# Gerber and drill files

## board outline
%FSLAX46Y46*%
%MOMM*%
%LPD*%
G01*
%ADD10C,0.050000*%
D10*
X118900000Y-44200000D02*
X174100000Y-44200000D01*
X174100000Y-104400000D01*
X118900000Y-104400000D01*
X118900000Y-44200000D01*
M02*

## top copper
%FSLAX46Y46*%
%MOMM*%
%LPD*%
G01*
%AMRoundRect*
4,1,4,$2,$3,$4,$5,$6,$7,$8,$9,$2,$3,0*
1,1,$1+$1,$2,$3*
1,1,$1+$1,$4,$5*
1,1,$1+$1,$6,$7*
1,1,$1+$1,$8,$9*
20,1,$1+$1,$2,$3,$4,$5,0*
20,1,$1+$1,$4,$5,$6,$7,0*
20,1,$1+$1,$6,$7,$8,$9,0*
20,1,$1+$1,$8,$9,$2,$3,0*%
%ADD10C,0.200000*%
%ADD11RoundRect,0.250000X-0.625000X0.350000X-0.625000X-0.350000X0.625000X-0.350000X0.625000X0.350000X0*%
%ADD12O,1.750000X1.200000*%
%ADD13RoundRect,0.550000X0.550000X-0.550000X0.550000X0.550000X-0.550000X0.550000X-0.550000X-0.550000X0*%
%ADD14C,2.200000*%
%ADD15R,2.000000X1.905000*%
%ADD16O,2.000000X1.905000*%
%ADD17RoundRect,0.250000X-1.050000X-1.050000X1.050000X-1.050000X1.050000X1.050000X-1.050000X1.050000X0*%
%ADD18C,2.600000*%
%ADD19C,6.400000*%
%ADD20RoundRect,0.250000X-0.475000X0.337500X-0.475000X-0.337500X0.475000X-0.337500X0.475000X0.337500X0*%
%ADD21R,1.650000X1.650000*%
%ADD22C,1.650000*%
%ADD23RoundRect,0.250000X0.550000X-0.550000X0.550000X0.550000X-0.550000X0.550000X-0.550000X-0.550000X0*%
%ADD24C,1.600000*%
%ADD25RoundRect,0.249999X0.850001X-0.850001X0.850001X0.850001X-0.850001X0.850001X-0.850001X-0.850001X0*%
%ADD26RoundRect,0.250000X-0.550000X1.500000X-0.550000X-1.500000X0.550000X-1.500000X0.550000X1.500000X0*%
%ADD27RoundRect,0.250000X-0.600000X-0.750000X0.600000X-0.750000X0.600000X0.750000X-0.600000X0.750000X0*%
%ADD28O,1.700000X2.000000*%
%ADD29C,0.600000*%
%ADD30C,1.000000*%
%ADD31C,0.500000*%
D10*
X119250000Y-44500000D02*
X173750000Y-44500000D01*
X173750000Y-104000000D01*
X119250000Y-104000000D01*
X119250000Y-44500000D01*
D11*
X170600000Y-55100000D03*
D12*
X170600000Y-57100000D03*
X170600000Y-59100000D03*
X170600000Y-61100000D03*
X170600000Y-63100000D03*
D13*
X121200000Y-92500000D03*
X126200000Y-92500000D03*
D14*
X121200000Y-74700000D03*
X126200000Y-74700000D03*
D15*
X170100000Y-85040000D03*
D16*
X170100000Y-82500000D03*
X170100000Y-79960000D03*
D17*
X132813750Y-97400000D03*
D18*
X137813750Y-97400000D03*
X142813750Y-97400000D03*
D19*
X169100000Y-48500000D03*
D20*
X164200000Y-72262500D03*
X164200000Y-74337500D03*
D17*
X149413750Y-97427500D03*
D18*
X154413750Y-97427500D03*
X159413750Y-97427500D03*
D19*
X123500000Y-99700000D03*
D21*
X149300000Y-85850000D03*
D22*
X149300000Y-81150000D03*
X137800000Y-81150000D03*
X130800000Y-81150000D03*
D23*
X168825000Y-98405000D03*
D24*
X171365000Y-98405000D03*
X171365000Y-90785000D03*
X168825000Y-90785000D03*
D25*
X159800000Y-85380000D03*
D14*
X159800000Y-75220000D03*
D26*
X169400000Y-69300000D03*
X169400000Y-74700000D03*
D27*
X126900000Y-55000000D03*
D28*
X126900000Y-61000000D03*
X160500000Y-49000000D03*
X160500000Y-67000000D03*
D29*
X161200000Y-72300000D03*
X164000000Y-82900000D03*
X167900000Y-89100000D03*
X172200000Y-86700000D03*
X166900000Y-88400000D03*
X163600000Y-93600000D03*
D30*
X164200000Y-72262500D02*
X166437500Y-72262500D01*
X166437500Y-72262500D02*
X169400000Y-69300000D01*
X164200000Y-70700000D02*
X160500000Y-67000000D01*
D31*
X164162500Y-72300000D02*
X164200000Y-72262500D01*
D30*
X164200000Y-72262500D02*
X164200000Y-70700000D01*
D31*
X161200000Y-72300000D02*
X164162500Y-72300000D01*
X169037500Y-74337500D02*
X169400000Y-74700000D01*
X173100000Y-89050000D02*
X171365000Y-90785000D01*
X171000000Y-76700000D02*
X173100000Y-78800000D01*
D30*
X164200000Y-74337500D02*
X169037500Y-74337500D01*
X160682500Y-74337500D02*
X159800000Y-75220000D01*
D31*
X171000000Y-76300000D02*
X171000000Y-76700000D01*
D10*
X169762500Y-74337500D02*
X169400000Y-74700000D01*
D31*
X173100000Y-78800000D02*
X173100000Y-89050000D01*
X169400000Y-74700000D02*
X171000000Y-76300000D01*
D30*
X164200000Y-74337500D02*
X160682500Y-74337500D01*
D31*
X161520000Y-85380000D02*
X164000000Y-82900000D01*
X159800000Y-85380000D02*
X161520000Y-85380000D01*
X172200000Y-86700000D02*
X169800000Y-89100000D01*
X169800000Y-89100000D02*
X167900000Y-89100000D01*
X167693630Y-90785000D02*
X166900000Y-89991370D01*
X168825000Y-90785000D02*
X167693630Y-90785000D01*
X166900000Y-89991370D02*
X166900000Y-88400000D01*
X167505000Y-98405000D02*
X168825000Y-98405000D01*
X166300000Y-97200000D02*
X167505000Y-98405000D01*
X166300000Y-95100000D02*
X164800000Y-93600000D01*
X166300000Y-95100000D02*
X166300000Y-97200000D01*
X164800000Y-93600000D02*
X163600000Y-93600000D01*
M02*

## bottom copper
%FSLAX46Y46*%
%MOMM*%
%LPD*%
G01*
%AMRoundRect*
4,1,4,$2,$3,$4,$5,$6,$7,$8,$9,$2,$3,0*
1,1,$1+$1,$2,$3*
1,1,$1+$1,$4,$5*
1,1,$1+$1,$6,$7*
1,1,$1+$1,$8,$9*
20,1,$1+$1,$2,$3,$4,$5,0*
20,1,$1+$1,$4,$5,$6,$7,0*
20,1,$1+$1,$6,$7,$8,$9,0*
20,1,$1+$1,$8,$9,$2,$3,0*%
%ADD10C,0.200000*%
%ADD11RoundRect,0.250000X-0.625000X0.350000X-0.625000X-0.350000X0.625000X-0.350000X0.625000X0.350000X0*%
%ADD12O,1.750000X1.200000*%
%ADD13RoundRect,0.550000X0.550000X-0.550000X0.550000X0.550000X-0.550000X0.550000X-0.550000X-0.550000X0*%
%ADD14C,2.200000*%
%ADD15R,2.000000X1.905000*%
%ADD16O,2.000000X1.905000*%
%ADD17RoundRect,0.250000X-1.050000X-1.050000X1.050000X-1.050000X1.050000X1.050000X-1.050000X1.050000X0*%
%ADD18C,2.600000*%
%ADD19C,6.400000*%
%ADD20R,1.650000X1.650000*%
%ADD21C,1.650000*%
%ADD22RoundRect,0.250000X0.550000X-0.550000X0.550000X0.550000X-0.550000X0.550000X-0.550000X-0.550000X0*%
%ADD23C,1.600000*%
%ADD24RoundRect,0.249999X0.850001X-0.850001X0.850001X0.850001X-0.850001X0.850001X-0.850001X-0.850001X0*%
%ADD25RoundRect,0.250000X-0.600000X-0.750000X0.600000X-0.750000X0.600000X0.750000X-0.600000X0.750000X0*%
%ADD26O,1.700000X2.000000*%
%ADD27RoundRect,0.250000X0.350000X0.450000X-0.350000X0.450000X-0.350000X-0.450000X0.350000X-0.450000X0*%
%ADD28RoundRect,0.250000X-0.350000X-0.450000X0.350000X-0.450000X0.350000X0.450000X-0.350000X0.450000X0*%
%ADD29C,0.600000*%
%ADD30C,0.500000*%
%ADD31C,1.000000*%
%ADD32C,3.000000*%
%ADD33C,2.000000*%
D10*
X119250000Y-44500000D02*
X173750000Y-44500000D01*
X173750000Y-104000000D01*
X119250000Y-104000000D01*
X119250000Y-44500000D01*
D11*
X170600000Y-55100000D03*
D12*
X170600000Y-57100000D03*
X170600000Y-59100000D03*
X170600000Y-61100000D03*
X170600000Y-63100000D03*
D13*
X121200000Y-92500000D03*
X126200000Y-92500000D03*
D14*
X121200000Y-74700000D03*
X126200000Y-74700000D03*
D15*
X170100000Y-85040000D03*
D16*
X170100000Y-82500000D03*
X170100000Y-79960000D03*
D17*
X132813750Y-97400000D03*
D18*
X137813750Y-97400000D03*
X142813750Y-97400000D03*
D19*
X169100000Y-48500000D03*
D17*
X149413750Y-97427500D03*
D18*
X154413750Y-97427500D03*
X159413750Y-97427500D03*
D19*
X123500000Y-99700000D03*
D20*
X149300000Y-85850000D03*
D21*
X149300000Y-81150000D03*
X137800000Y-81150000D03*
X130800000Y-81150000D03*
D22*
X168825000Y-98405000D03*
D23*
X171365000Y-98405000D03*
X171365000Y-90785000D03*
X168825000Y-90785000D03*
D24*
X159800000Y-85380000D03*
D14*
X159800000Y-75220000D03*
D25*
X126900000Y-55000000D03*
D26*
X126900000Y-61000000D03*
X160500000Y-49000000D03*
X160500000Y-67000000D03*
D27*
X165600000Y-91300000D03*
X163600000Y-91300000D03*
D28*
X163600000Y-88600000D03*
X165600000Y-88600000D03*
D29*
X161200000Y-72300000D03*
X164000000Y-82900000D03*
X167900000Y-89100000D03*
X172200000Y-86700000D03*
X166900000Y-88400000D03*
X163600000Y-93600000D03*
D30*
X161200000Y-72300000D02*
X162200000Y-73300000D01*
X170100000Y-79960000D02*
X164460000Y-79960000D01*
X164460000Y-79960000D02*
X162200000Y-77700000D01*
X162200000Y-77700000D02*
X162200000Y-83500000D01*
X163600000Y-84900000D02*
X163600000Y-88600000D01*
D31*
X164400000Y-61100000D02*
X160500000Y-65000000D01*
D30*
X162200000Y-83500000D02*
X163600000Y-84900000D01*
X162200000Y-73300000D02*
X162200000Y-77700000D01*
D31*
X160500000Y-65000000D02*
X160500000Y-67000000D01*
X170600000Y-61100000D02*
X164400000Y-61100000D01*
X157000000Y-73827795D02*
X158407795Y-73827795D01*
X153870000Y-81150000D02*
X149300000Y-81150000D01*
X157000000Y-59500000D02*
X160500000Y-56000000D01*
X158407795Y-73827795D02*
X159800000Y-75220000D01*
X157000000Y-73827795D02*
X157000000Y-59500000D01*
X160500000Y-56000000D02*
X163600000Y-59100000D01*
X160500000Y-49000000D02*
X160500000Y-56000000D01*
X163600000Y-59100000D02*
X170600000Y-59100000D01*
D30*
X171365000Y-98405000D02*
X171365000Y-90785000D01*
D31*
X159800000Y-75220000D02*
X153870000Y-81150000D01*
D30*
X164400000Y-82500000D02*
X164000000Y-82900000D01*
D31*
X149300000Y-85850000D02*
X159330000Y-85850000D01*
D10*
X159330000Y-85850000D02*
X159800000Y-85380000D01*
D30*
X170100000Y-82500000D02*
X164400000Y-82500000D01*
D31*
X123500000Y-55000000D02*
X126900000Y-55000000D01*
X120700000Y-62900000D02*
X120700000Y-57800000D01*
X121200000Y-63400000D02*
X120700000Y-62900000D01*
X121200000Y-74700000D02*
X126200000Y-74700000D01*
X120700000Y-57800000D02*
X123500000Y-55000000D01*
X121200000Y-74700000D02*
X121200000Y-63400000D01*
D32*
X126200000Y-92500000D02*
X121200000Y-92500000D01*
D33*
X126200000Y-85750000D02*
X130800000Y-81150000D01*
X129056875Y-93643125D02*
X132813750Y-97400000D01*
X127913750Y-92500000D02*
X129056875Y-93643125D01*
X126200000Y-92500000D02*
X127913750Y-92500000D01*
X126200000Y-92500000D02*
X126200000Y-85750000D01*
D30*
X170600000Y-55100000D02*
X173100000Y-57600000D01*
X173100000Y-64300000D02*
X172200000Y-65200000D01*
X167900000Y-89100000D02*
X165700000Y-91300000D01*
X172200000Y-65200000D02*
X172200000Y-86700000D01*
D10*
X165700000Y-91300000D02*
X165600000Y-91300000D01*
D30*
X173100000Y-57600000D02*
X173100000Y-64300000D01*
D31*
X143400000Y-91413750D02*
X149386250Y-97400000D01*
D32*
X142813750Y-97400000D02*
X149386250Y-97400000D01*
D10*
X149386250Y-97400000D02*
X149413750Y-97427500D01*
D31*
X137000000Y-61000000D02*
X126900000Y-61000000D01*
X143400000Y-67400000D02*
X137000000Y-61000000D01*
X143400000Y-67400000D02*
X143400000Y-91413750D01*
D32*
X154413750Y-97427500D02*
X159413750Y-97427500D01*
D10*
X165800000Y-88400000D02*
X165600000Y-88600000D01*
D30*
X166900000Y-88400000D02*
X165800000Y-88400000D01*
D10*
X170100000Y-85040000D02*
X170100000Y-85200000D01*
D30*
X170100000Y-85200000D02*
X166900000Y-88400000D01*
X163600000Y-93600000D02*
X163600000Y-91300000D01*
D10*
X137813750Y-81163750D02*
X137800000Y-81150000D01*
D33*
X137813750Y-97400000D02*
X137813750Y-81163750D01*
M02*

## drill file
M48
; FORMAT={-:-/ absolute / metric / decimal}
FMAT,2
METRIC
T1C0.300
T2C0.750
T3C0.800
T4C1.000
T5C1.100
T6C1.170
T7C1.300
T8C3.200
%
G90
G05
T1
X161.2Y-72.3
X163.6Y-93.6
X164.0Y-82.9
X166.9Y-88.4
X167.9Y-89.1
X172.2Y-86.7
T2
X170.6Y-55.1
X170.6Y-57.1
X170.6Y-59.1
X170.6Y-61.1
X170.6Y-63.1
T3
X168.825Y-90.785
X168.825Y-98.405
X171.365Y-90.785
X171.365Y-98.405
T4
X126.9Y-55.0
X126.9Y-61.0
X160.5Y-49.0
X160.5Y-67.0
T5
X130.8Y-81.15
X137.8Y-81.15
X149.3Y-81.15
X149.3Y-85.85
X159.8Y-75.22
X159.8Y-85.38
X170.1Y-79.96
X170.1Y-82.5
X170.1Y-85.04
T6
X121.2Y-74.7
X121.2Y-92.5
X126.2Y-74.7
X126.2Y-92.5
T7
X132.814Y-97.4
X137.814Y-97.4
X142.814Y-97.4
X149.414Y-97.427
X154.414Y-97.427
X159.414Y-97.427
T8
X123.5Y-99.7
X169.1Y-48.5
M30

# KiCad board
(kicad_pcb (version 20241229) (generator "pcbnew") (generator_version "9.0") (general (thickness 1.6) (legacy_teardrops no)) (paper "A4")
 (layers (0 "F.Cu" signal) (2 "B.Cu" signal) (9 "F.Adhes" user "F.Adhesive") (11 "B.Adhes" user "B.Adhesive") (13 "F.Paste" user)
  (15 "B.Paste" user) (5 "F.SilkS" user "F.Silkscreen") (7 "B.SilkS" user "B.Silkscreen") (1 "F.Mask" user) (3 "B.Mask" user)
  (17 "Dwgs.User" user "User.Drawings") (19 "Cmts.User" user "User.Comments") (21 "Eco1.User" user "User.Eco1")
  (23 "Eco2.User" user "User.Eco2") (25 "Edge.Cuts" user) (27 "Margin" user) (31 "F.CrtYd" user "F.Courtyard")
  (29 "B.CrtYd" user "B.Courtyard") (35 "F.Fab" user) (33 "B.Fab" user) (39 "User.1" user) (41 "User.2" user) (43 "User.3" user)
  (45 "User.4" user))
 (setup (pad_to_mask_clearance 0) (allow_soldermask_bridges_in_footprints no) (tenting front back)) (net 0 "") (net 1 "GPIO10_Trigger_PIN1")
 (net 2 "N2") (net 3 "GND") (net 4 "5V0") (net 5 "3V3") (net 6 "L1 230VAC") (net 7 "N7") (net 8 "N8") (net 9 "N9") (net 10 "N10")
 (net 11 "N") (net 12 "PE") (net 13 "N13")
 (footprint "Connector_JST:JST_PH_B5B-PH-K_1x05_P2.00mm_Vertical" (layer "F.Cu") (at 170.6 55.1 -90)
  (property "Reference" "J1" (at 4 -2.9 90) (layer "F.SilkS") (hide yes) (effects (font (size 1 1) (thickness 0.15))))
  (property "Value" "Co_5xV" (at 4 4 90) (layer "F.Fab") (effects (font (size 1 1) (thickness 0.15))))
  (pad "1" thru_hole roundrect (at 0 0 270) (size 1.2 1.75) (drill 0.75) (layers "*.Cu" "*.Mask") (remove_unused_layers no)
   (roundrect_rratio 0.208333) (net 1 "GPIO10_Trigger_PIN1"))
  (pad "2" thru_hole oval (at 2 0 270) (size 1.2 1.75) (drill 0.75) (layers "*.Cu" "*.Mask") (remove_unused_layers no) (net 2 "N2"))
  (pad "3" thru_hole oval (at 4 0 270) (size 1.2 1.75) (drill 0.75) (layers "*.Cu" "*.Mask") (remove_unused_layers no) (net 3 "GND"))
  (pad "4" thru_hole oval (at 6 0 270) (size 1.2 1.75) (drill 0.75) (layers "*.Cu" "*.Mask") (remove_unused_layers no) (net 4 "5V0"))
  (pad "5" thru_hole oval (at 8 0 270) (size 1.2 1.75) (drill 0.75) (layers "*.Cu" "*.Mask") (remove_unused_layers no) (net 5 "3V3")))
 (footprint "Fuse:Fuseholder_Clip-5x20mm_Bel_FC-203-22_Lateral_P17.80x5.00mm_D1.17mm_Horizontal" (layer "F.Cu") (at 121.2 92.5 90)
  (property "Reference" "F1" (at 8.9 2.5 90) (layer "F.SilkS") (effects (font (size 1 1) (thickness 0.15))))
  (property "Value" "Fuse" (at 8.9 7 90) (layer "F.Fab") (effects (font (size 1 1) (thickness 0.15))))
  (pad "1" thru_hole roundrect (at 0 0 90) (size 2.2 2.2) (drill 1.17) (layers "*.Cu" "*.Mask") (remove_unused_layers no)
   (roundrect_rratio 0.25) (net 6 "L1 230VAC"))
  (pad "1" thru_hole roundrect (at 0 5 90) (size 2.2 2.2) (drill 1.17) (layers "*.Cu" "*.Mask") (remove_unused_layers no)
   (roundrect_rratio 0.25) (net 6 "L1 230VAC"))
  (pad "2" thru_hole circle (at 17.8 0 90) (size 2.2 2.2) (drill 1.17) (layers "*.Cu" "*.Mask") (remove_unused_layers no) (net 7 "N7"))
  (pad "2" thru_hole circle (at 17.8 5 90) (size 2.2 2.2) (drill 1.17) (layers "*.Cu" "*.Mask") (remove_unused_layers no) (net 7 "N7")))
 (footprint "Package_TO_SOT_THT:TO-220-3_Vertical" (layer "F.Cu") (at 170.1 85.04 90)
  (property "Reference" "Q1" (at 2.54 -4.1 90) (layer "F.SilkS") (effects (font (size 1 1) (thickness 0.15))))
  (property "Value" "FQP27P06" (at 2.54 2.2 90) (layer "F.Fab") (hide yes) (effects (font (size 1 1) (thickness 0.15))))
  (pad "1" thru_hole rect (at 0 0 90) (size 1.905 2) (drill 1.1) (layers "*.Cu" "*.Mask") (remove_unused_layers no) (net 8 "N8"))
  (pad "2" thru_hole oval (at 2.54 0 90) (size 1.905 2) (drill 1.1) (layers "*.Cu" "*.Mask") (remove_unused_layers no) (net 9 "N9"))
  (pad "3" thru_hole oval (at 5.08 0 90) (size 1.905 2) (drill 1.1) (layers "*.Cu" "*.Mask") (remove_unused_layers no) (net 4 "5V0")))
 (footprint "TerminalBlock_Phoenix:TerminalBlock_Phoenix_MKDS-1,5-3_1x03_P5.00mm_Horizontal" (layer "F.Cu") (at 132.81375 97.4)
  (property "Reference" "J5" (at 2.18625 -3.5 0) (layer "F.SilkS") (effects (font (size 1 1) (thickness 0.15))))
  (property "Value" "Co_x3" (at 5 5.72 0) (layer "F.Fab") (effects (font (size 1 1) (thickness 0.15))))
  (pad "1" thru_hole roundrect (at 0 0) (size 2.6 2.6) (drill 1.3) (layers "*.Cu" "*.Mask") (remove_unused_layers no)
   (roundrect_rratio 0.096154) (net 6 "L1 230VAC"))
  (pad "2" thru_hole circle (at 5 0) (size 2.6 2.6) (drill 1.3) (layers "*.Cu" "*.Mask") (remove_unused_layers no) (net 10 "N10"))
  (pad "3" thru_hole circle (at 10 0) (size 2.6 2.6) (drill 1.3) (layers "*.Cu" "*.Mask") (remove_unused_layers no) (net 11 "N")))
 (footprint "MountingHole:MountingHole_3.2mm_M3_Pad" (layer "F.Cu") (at 169.1 48.5)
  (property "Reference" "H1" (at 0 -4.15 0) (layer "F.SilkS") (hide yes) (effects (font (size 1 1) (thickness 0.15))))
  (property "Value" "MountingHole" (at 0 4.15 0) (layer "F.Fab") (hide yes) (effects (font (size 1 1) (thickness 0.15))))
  (pad "1" thru_hole circle (at 0 0) (size 6.4 6.4) (drill 3.2) (layers "*.Cu" "*.Mask") (remove_unused_layers no) (zone_connect 2)))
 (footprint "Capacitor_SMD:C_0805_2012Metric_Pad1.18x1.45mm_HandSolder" (layer "F.Cu") (at 164.2 73.3 -90)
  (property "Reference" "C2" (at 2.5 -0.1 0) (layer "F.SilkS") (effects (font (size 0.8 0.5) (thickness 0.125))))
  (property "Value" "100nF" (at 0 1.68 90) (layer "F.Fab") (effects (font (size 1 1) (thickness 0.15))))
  (pad "1" smd roundrect (at -1.0375 0 270) (size 1.175 1.45) (layers "F.Cu" "F.Mask" "F.Paste") (roundrect_rratio 0.212766) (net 4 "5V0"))
  (pad "2" smd roundrect (at 1.0375 0 270) (size 1.175 1.45) (layers "F.Cu" "F.Mask" "F.Paste") (roundrect_rratio 0.212766) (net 3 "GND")))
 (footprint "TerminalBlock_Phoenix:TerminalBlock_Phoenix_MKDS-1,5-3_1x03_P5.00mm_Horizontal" (layer "F.Cu") (at 149.41375 97.4275)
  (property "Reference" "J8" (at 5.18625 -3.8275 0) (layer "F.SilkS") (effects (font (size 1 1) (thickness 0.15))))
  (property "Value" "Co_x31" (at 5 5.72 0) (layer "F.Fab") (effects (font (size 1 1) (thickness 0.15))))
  (pad "1" thru_hole roundrect (at 0 0) (size 2.6 2.6) (drill 1.3) (layers "*.Cu" "*.Mask") (remove_unused_layers no)
   (roundrect_rratio 0.096154) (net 11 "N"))
  (pad "2" thru_hole circle (at 5 0) (size 2.6 2.6) (drill 1.3) (layers "*.Cu" "*.Mask") (remove_unused_layers no) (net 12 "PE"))
  (pad "3" thru_hole circle (at 10 0) (size 2.6 2.6) (drill 1.3) (layers "*.Cu" "*.Mask") (remove_unused_layers no) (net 12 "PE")))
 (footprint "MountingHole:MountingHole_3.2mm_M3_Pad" (layer "F.Cu") (at 123.5 99.7)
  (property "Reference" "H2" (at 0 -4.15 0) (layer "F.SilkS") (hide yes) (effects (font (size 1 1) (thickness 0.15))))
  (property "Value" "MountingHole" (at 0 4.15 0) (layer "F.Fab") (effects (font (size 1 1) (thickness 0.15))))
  (pad "1" thru_hole circle (at 0 0) (size 6.4 6.4) (drill 3.2) (layers "*.Cu" "*.Mask") (remove_unused_layers no) (zone_connect 2)))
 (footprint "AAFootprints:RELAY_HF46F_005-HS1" (layer "F.Cu") (at 140.1 83.5 180)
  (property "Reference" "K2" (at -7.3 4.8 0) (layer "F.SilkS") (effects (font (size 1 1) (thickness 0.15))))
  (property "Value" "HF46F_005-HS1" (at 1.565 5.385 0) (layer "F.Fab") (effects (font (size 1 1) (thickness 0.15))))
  (pad "1" thru_hole rect (at -9.2 -2.35 180) (size 1.65 1.65) (drill 1.1) (layers "*.Cu" "*.Mask") (remove_unused_layers no) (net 9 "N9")
   (solder_mask_margin 0.102))
  (pad "2" thru_hole circle (at -9.2 2.35 180) (size 1.65 1.65) (drill 1.1) (layers "*.Cu" "*.Mask") (remove_unused_layers no) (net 3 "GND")
   (solder_mask_margin 0.102))
  (pad "3" thru_hole circle (at 2.3 2.35 180) (size 1.65 1.65) (drill 1.1) (layers "*.Cu" "*.Mask") (remove_unused_layers no) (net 10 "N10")
   (solder_mask_margin 0.102))
  (pad "4" thru_hole circle (at 9.3 2.35 180) (size 1.65 1.65) (drill 1.1) (layers "*.Cu" "*.Mask") (remove_unused_layers no)
   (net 6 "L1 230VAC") (solder_mask_margin 0.102)))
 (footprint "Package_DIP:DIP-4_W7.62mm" (layer "F.Cu") (at 168.825 98.405 90)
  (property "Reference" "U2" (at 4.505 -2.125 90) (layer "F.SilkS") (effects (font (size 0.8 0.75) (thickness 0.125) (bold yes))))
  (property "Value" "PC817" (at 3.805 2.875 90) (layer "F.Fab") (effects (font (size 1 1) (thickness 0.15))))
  (pad "1" thru_hole roundrect (at 0 0 90) (size 1.6 1.6) (drill 0.8) (layers "*.Cu" "*.Mask") (remove_unused_layers no)
   (roundrect_rratio 0.15625) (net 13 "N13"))
  (pad "2" thru_hole circle (at 0 2.54 90) (size 1.6 1.6) (drill 0.8) (layers "*.Cu" "*.Mask") (remove_unused_layers no) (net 3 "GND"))
  (pad "3" thru_hole circle (at 7.62 2.54 90) (size 1.6 1.6) (drill 0.8) (layers "*.Cu" "*.Mask") (remove_unused_layers no) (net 3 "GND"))
  (pad "4" thru_hole circle (at 7.62 0 90) (size 1.6 1.6) (drill 0.8) (layers "*.Cu" "*.Mask") (remove_unused_layers no) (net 8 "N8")))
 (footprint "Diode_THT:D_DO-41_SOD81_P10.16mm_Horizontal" (layer "F.Cu") (at 159.8 85.38 90)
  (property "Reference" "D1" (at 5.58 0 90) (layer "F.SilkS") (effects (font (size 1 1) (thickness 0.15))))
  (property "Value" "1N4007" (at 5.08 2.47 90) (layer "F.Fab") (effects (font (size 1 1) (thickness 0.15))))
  (pad "1" thru_hole roundrect (at 0 0 90) (size 2.2 2.2) (drill 1.1) (layers "*.Cu" "*.Mask") (remove_unused_layers no)
   (roundrect_rratio 0.113636) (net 9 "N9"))
  (pad "2" thru_hole circle (at 10.16 0 90) (size 2.2 2.2) (drill 1.1) (layers "*.Cu" "*.Mask") (remove_unused_layers no) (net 3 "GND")))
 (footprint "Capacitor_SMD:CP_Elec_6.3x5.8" (layer "F.Cu") (at 169.4 72 -90)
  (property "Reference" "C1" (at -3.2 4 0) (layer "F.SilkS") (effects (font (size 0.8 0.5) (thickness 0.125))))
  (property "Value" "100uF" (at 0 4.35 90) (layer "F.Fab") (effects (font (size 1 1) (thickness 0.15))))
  (pad "1" smd roundrect (at -2.7 0 270) (size 3.5 1.6) (layers "F.Cu" "F.Mask" "F.Paste") (roundrect_rratio 0.15625) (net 4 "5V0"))
  (pad "2" smd roundrect (at 2.7 0 270) (size 3.5 1.6) (layers "F.Cu" "F.Mask" "F.Paste") (roundrect_rratio 0.15625) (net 3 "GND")))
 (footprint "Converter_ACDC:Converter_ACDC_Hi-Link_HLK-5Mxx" (layer "F.Cu") (at 126.9 55)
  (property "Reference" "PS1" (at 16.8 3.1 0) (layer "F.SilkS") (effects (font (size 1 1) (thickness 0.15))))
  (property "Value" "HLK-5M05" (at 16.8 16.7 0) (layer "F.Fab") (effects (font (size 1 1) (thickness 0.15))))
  (pad "1" thru_hole roundrect (at 0 0) (size 1.7 2) (drill 1) (layers "*.Cu" "*.Mask") (remove_unused_layers no)
   (roundrect_rratio 0.147059) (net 7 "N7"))
  (pad "2" thru_hole oval (at 0 6) (size 1.7 2) (drill 1) (layers "*.Cu" "*.Mask") (remove_unused_layers no) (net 11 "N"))
  (pad "3" thru_hole oval (at 33.6 -6) (size 1.7 2) (drill 1) (layers "*.Cu" "*.Mask") (remove_unused_layers no) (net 3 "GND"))
  (pad "4" thru_hole oval (at 33.6 12) (size 1.7 2) (drill 1) (layers "*.Cu" "*.Mask") (remove_unused_layers no) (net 4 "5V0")))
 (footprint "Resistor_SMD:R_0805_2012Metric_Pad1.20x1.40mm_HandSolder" (layer "B.Cu") (at 164.6 91.3 180)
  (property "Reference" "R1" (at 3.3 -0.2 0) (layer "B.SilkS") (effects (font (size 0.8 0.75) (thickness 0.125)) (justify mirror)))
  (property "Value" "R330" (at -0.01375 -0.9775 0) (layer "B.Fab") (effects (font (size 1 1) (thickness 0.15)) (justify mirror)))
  (pad "1" smd roundrect (at -1 0 180) (size 1.2 1.4) (layers "B.Cu" "B.Mask" "B.Paste") (roundrect_rratio 0.208333)
   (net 1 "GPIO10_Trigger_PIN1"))
  (pad "2" smd roundrect (at 1 0 180) (size 1.2 1.4) (layers "B.Cu" "B.Mask" "B.Paste") (roundrect_rratio 0.208333) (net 13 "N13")))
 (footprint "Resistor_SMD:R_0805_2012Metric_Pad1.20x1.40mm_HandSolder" (layer "B.Cu") (at 164.6 88.6)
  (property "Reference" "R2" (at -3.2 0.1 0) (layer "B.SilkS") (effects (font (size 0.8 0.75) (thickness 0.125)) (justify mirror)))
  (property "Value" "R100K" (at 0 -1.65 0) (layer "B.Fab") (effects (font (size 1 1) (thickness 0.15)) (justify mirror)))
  (pad "1" smd roundrect (at -1 0) (size 1.2 1.4) (layers "B.Cu" "B.Mask" "B.Paste") (roundrect_rratio 0.208333) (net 4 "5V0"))
  (pad "2" smd roundrect (at 1 0) (size 1.2 1.4) (layers "B.Cu" "B.Mask" "B.Paste") (roundrect_rratio 0.208333) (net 8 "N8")))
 (gr_rect (start 119.25 44.5) (end 173.75 104) (stroke (width 0.2) (type default)) (fill no) (layer "F.Cu") (net 10))
 (gr_rect (start 119.25 44.5) (end 173.75 104) (stroke (width 0.2) (type default)) (fill no) (layer "B.Cu") (net 10))
 (gr_rect (start 118.9 44.2) (end 174.1 104.4) (stroke (width 0.05) (type solid)) (fill no) (layer "Edge.Cuts"))
 (segment (start 164.2 72.2625) (end 166.4375 72.2625) (width 1) (layer "F.Cu") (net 4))
 (segment (start 166.4375 72.2625) (end 169.4 69.3) (width 1) (layer "F.Cu") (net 4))
 (segment (start 164.2 70.7) (end 160.5 67) (width 1) (layer "F.Cu") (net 4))
 (segment (start 164.1625 72.3) (end 164.2 72.2625) (width 0.5) (layer "F.Cu") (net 4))
 (segment (start 164.2 72.2625) (end 164.2 70.7) (width 1) (layer "F.Cu") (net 4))
 (segment (start 161.2 72.3) (end 164.1625 72.3) (width 0.5) (layer "F.Cu") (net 4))
 (via (at 161.2 72.3) (size 0.6) (drill 0.3) (layers "F.Cu" "B.Cu") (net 4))
 (segment (start 161.2 72.3) (end 162.2 73.3) (width 0.5) (layer "B.Cu") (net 4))
 (segment (start 170.1 79.96) (end 164.46 79.96) (width 0.5) (layer "B.Cu") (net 4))
 (segment (start 164.46 79.96) (end 162.2 77.7) (width 0.5) (layer "B.Cu") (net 4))
 (segment (start 162.2 77.7) (end 162.2 83.5) (width 0.5) (layer "B.Cu") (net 4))
 (segment (start 163.6 84.9) (end 163.6 88.6) (width 0.5) (layer "B.Cu") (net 4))
 (segment (start 164.4 61.1) (end 160.5 65) (width 1) (layer "B.Cu") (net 4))
 (segment (start 162.2 83.5) (end 163.6 84.9) (width 0.5) (layer "B.Cu") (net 4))
 (segment (start 162.2 73.3) (end 162.2 77.7) (width 0.5) (layer "B.Cu") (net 4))
 (segment (start 160.5 65) (end 160.5 67) (width 1) (layer "B.Cu") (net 4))
 (segment (start 170.6 61.1) (end 164.4 61.1) (width 1) (layer "B.Cu") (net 4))
 (segment (start 169.0375 74.3375) (end 169.4 74.7) (width 0.5) (layer "F.Cu") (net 3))
 (segment (start 173.1 89.05) (end 171.365 90.785) (width 0.5) (layer "F.Cu") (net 3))
 (segment (start 171 76.7) (end 173.1 78.8) (width 0.5) (layer "F.Cu") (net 3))
 (segment (start 164.2 74.3375) (end 169.0375 74.3375) (width 1) (layer "F.Cu") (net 3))
 (segment (start 160.6825 74.3375) (end 159.8 75.22) (width 1) (layer "F.Cu") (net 3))
 (segment (start 171 76.3) (end 171 76.7) (width 0.5) (layer "F.Cu") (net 3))
 (segment (start 169.7625 74.3375) (end 169.4 74.7) (width 0.2) (layer "F.Cu") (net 3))
 (segment (start 173.1 78.8) (end 173.1 89.05) (width 0.5) (layer "F.Cu") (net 3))
 (segment (start 169.4 74.7) (end 171 76.3) (width 0.5) (layer "F.Cu") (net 3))
 (segment (start 164.2 74.3375) (end 160.6825 74.3375) (width 1) (layer "F.Cu") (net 3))
 (segment (start 157 73.827795) (end 158.407795 73.827795) (width 1) (layer "B.Cu") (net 3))
 (segment (start 153.87 81.15) (end 149.3 81.15) (width 1) (layer "B.Cu") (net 3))
 (segment (start 157 59.5) (end 160.5 56) (width 1) (layer "B.Cu") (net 3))
 (segment (start 158.407795 73.827795) (end 159.8 75.22) (width 1) (layer "B.Cu") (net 3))
 (segment (start 157 73.827795) (end 157 59.5) (width 1) (layer "B.Cu") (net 3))
 (segment (start 160.5 56) (end 163.6 59.1) (width 1) (layer "B.Cu") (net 3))
 (segment (start 160.5 49) (end 160.5 56) (width 1) (layer "B.Cu") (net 3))
 (segment (start 163.6 59.1) (end 170.6 59.1) (width 1) (layer "B.Cu") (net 3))
 (segment (start 171.365 98.405) (end 171.365 90.785) (width 0.5) (layer "B.Cu") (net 3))
 (segment (start 159.8 75.22) (end 153.87 81.15) (width 1) (layer "B.Cu") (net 3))
 (segment (start 161.52 85.38) (end 164 82.9) (width 0.5) (layer "F.Cu") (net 9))
 (segment (start 159.8 85.38) (end 161.52 85.38) (width 0.5) (layer "F.Cu") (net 9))
 (via (at 164 82.9) (size 0.6) (drill 0.3) (layers "F.Cu" "B.Cu") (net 9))
 (segment (start 164.4 82.5) (end 164 82.9) (width 0.5) (layer "B.Cu") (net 9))
 (segment (start 149.3 85.85) (end 159.33 85.85) (width 1) (layer "B.Cu") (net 9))
 (segment (start 159.33 85.85) (end 159.8 85.38) (width 0.2) (layer "B.Cu") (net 9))
 (segment (start 170.1 82.5) (end 164.4 82.5) (width 0.5) (layer "B.Cu") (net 9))
 (segment (start 123.5 55) (end 126.9 55) (width 1) (layer "B.Cu") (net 7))
 (segment (start 120.7 62.9) (end 120.7 57.8) (width 1) (layer "B.Cu") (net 7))
 (segment (start 121.2 63.4) (end 120.7 62.9) (width 1) (layer "B.Cu") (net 7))
 (segment (start 121.2 74.7) (end 126.2 74.7) (width 1) (layer "B.Cu") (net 7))
 (segment (start 120.7 57.8) (end 123.5 55) (width 1) (layer "B.Cu") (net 7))
 (segment (start 121.2 74.7) (end 121.2 63.4) (width 1) (layer "B.Cu") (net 7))
 (segment (start 126.2 92.5) (end 121.2 92.5) (width 3) (layer "B.Cu") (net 6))
 (segment (start 126.2 85.75) (end 130.8 81.15) (width 2) (layer "B.Cu") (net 6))
 (segment (start 129.056875 93.643125) (end 132.81375 97.4) (width 2) (layer "B.Cu") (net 6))
 (segment (start 127.91375 92.5) (end 129.056875 93.643125) (width 2) (layer "B.Cu") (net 6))
 (segment (start 126.2 92.5) (end 127.91375 92.5) (width 2) (layer "B.Cu") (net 6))
 (segment (start 126.2 92.5) (end 126.2 85.75) (width 2) (layer "B.Cu") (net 6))
 (segment (start 172.2 86.7) (end 169.8 89.1) (width 0.5) (layer "F.Cu") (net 1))
 (segment (start 169.8 89.1) (end 167.9 89.1) (width 0.5) (layer "F.Cu") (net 1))
 (via (at 167.9 89.1) (size 0.6) (drill 0.3) (layers "F.Cu" "B.Cu") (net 1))
 (via (at 172.2 86.7) (size 0.6) (drill 0.3) (layers "F.Cu" "B.Cu") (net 1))
 (segment (start 170.6 55.1) (end 173.1 57.6) (width 0.5) (layer "B.Cu") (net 1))
 (segment (start 173.1 64.3) (end 172.2 65.2) (width 0.5) (layer "B.Cu") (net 1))
 (segment (start 167.9 89.1) (end 165.7 91.3) (width 0.5) (layer "B.Cu") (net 1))
 (segment (start 172.2 65.2) (end 172.2 86.7) (width 0.5) (layer "B.Cu") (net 1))
 (segment (start 165.7 91.3) (end 165.6 91.3) (width 0.2) (layer "B.Cu") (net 1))
 (segment (start 173.1 57.6) (end 173.1 64.3) (width 0.5) (layer "B.Cu") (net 1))
 (segment (start 143.4 91.41375) (end 149.38625 97.4) (width 1) (layer "B.Cu") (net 11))
 (segment (start 142.81375 97.4) (end 149.38625 97.4) (width 3) (layer "B.Cu") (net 11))
 (segment (start 149.38625 97.4) (end 149.41375 97.4275) (width 0.2) (layer "B.Cu") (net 11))
 (segment (start 137 61) (end 126.9 61) (width 1) (layer "B.Cu") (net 11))
 (segment (start 143.4 67.4) (end 137 61) (width 1) (layer "B.Cu") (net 11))
 (segment (start 143.4 67.4) (end 143.4 91.41375) (width 1) (layer "B.Cu") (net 11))
 (segment (start 154.41375 97.4275) (end 159.41375 97.4275) (width 3) (layer "B.Cu") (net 12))
 (segment (start 167.69363 90.785) (end 166.9 89.99137) (width 0.5) (layer "F.Cu") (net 8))
 (segment (start 168.825 90.785) (end 167.69363 90.785) (width 0.5) (layer "F.Cu") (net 8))
 (segment (start 166.9 89.99137) (end 166.9 88.4) (width 0.5) (layer "F.Cu") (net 8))
 (via (at 166.9 88.4) (size 0.6) (drill 0.3) (layers "F.Cu" "B.Cu") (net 8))
 (segment (start 165.8 88.4) (end 165.6 88.6) (width 0.2) (layer "B.Cu") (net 8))
 (segment (start 166.9 88.4) (end 165.8 88.4) (width 0.5) (layer "B.Cu") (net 8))
 (segment (start 170.1 85.04) (end 170.1 85.2) (width 0.2) (layer "B.Cu") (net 8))
 (segment (start 170.1 85.2) (end 166.9 88.4) (width 0.5) (layer "B.Cu") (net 8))
 (segment (start 167.505 98.405) (end 168.825 98.405) (width 0.5) (layer "F.Cu") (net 13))
 (segment (start 166.3 97.2) (end 167.505 98.405) (width 0.5) (layer "F.Cu") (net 13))
 (segment (start 166.3 95.1) (end 164.8 93.6) (width 0.5) (layer "F.Cu") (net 13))
 (segment (start 166.3 95.1) (end 166.3 97.2) (width 0.5) (layer "F.Cu") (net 13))
 (segment (start 164.8 93.6) (end 163.6 93.6) (width 0.5) (layer "F.Cu") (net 13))
 (via (at 163.6 93.6) (size 0.6) (drill 0.3) (layers "F.Cu" "B.Cu") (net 13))
 (segment (start 163.6 93.6) (end 163.6 91.3) (width 0.5) (layer "B.Cu") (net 13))
 (segment (start 137.81375 81.16375) (end 137.8 81.15) (width 0.2) (layer "B.Cu") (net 10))
 (segment (start 137.81375 97.4) (end 137.81375 81.16375) (width 2) (layer "B.Cu") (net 10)))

